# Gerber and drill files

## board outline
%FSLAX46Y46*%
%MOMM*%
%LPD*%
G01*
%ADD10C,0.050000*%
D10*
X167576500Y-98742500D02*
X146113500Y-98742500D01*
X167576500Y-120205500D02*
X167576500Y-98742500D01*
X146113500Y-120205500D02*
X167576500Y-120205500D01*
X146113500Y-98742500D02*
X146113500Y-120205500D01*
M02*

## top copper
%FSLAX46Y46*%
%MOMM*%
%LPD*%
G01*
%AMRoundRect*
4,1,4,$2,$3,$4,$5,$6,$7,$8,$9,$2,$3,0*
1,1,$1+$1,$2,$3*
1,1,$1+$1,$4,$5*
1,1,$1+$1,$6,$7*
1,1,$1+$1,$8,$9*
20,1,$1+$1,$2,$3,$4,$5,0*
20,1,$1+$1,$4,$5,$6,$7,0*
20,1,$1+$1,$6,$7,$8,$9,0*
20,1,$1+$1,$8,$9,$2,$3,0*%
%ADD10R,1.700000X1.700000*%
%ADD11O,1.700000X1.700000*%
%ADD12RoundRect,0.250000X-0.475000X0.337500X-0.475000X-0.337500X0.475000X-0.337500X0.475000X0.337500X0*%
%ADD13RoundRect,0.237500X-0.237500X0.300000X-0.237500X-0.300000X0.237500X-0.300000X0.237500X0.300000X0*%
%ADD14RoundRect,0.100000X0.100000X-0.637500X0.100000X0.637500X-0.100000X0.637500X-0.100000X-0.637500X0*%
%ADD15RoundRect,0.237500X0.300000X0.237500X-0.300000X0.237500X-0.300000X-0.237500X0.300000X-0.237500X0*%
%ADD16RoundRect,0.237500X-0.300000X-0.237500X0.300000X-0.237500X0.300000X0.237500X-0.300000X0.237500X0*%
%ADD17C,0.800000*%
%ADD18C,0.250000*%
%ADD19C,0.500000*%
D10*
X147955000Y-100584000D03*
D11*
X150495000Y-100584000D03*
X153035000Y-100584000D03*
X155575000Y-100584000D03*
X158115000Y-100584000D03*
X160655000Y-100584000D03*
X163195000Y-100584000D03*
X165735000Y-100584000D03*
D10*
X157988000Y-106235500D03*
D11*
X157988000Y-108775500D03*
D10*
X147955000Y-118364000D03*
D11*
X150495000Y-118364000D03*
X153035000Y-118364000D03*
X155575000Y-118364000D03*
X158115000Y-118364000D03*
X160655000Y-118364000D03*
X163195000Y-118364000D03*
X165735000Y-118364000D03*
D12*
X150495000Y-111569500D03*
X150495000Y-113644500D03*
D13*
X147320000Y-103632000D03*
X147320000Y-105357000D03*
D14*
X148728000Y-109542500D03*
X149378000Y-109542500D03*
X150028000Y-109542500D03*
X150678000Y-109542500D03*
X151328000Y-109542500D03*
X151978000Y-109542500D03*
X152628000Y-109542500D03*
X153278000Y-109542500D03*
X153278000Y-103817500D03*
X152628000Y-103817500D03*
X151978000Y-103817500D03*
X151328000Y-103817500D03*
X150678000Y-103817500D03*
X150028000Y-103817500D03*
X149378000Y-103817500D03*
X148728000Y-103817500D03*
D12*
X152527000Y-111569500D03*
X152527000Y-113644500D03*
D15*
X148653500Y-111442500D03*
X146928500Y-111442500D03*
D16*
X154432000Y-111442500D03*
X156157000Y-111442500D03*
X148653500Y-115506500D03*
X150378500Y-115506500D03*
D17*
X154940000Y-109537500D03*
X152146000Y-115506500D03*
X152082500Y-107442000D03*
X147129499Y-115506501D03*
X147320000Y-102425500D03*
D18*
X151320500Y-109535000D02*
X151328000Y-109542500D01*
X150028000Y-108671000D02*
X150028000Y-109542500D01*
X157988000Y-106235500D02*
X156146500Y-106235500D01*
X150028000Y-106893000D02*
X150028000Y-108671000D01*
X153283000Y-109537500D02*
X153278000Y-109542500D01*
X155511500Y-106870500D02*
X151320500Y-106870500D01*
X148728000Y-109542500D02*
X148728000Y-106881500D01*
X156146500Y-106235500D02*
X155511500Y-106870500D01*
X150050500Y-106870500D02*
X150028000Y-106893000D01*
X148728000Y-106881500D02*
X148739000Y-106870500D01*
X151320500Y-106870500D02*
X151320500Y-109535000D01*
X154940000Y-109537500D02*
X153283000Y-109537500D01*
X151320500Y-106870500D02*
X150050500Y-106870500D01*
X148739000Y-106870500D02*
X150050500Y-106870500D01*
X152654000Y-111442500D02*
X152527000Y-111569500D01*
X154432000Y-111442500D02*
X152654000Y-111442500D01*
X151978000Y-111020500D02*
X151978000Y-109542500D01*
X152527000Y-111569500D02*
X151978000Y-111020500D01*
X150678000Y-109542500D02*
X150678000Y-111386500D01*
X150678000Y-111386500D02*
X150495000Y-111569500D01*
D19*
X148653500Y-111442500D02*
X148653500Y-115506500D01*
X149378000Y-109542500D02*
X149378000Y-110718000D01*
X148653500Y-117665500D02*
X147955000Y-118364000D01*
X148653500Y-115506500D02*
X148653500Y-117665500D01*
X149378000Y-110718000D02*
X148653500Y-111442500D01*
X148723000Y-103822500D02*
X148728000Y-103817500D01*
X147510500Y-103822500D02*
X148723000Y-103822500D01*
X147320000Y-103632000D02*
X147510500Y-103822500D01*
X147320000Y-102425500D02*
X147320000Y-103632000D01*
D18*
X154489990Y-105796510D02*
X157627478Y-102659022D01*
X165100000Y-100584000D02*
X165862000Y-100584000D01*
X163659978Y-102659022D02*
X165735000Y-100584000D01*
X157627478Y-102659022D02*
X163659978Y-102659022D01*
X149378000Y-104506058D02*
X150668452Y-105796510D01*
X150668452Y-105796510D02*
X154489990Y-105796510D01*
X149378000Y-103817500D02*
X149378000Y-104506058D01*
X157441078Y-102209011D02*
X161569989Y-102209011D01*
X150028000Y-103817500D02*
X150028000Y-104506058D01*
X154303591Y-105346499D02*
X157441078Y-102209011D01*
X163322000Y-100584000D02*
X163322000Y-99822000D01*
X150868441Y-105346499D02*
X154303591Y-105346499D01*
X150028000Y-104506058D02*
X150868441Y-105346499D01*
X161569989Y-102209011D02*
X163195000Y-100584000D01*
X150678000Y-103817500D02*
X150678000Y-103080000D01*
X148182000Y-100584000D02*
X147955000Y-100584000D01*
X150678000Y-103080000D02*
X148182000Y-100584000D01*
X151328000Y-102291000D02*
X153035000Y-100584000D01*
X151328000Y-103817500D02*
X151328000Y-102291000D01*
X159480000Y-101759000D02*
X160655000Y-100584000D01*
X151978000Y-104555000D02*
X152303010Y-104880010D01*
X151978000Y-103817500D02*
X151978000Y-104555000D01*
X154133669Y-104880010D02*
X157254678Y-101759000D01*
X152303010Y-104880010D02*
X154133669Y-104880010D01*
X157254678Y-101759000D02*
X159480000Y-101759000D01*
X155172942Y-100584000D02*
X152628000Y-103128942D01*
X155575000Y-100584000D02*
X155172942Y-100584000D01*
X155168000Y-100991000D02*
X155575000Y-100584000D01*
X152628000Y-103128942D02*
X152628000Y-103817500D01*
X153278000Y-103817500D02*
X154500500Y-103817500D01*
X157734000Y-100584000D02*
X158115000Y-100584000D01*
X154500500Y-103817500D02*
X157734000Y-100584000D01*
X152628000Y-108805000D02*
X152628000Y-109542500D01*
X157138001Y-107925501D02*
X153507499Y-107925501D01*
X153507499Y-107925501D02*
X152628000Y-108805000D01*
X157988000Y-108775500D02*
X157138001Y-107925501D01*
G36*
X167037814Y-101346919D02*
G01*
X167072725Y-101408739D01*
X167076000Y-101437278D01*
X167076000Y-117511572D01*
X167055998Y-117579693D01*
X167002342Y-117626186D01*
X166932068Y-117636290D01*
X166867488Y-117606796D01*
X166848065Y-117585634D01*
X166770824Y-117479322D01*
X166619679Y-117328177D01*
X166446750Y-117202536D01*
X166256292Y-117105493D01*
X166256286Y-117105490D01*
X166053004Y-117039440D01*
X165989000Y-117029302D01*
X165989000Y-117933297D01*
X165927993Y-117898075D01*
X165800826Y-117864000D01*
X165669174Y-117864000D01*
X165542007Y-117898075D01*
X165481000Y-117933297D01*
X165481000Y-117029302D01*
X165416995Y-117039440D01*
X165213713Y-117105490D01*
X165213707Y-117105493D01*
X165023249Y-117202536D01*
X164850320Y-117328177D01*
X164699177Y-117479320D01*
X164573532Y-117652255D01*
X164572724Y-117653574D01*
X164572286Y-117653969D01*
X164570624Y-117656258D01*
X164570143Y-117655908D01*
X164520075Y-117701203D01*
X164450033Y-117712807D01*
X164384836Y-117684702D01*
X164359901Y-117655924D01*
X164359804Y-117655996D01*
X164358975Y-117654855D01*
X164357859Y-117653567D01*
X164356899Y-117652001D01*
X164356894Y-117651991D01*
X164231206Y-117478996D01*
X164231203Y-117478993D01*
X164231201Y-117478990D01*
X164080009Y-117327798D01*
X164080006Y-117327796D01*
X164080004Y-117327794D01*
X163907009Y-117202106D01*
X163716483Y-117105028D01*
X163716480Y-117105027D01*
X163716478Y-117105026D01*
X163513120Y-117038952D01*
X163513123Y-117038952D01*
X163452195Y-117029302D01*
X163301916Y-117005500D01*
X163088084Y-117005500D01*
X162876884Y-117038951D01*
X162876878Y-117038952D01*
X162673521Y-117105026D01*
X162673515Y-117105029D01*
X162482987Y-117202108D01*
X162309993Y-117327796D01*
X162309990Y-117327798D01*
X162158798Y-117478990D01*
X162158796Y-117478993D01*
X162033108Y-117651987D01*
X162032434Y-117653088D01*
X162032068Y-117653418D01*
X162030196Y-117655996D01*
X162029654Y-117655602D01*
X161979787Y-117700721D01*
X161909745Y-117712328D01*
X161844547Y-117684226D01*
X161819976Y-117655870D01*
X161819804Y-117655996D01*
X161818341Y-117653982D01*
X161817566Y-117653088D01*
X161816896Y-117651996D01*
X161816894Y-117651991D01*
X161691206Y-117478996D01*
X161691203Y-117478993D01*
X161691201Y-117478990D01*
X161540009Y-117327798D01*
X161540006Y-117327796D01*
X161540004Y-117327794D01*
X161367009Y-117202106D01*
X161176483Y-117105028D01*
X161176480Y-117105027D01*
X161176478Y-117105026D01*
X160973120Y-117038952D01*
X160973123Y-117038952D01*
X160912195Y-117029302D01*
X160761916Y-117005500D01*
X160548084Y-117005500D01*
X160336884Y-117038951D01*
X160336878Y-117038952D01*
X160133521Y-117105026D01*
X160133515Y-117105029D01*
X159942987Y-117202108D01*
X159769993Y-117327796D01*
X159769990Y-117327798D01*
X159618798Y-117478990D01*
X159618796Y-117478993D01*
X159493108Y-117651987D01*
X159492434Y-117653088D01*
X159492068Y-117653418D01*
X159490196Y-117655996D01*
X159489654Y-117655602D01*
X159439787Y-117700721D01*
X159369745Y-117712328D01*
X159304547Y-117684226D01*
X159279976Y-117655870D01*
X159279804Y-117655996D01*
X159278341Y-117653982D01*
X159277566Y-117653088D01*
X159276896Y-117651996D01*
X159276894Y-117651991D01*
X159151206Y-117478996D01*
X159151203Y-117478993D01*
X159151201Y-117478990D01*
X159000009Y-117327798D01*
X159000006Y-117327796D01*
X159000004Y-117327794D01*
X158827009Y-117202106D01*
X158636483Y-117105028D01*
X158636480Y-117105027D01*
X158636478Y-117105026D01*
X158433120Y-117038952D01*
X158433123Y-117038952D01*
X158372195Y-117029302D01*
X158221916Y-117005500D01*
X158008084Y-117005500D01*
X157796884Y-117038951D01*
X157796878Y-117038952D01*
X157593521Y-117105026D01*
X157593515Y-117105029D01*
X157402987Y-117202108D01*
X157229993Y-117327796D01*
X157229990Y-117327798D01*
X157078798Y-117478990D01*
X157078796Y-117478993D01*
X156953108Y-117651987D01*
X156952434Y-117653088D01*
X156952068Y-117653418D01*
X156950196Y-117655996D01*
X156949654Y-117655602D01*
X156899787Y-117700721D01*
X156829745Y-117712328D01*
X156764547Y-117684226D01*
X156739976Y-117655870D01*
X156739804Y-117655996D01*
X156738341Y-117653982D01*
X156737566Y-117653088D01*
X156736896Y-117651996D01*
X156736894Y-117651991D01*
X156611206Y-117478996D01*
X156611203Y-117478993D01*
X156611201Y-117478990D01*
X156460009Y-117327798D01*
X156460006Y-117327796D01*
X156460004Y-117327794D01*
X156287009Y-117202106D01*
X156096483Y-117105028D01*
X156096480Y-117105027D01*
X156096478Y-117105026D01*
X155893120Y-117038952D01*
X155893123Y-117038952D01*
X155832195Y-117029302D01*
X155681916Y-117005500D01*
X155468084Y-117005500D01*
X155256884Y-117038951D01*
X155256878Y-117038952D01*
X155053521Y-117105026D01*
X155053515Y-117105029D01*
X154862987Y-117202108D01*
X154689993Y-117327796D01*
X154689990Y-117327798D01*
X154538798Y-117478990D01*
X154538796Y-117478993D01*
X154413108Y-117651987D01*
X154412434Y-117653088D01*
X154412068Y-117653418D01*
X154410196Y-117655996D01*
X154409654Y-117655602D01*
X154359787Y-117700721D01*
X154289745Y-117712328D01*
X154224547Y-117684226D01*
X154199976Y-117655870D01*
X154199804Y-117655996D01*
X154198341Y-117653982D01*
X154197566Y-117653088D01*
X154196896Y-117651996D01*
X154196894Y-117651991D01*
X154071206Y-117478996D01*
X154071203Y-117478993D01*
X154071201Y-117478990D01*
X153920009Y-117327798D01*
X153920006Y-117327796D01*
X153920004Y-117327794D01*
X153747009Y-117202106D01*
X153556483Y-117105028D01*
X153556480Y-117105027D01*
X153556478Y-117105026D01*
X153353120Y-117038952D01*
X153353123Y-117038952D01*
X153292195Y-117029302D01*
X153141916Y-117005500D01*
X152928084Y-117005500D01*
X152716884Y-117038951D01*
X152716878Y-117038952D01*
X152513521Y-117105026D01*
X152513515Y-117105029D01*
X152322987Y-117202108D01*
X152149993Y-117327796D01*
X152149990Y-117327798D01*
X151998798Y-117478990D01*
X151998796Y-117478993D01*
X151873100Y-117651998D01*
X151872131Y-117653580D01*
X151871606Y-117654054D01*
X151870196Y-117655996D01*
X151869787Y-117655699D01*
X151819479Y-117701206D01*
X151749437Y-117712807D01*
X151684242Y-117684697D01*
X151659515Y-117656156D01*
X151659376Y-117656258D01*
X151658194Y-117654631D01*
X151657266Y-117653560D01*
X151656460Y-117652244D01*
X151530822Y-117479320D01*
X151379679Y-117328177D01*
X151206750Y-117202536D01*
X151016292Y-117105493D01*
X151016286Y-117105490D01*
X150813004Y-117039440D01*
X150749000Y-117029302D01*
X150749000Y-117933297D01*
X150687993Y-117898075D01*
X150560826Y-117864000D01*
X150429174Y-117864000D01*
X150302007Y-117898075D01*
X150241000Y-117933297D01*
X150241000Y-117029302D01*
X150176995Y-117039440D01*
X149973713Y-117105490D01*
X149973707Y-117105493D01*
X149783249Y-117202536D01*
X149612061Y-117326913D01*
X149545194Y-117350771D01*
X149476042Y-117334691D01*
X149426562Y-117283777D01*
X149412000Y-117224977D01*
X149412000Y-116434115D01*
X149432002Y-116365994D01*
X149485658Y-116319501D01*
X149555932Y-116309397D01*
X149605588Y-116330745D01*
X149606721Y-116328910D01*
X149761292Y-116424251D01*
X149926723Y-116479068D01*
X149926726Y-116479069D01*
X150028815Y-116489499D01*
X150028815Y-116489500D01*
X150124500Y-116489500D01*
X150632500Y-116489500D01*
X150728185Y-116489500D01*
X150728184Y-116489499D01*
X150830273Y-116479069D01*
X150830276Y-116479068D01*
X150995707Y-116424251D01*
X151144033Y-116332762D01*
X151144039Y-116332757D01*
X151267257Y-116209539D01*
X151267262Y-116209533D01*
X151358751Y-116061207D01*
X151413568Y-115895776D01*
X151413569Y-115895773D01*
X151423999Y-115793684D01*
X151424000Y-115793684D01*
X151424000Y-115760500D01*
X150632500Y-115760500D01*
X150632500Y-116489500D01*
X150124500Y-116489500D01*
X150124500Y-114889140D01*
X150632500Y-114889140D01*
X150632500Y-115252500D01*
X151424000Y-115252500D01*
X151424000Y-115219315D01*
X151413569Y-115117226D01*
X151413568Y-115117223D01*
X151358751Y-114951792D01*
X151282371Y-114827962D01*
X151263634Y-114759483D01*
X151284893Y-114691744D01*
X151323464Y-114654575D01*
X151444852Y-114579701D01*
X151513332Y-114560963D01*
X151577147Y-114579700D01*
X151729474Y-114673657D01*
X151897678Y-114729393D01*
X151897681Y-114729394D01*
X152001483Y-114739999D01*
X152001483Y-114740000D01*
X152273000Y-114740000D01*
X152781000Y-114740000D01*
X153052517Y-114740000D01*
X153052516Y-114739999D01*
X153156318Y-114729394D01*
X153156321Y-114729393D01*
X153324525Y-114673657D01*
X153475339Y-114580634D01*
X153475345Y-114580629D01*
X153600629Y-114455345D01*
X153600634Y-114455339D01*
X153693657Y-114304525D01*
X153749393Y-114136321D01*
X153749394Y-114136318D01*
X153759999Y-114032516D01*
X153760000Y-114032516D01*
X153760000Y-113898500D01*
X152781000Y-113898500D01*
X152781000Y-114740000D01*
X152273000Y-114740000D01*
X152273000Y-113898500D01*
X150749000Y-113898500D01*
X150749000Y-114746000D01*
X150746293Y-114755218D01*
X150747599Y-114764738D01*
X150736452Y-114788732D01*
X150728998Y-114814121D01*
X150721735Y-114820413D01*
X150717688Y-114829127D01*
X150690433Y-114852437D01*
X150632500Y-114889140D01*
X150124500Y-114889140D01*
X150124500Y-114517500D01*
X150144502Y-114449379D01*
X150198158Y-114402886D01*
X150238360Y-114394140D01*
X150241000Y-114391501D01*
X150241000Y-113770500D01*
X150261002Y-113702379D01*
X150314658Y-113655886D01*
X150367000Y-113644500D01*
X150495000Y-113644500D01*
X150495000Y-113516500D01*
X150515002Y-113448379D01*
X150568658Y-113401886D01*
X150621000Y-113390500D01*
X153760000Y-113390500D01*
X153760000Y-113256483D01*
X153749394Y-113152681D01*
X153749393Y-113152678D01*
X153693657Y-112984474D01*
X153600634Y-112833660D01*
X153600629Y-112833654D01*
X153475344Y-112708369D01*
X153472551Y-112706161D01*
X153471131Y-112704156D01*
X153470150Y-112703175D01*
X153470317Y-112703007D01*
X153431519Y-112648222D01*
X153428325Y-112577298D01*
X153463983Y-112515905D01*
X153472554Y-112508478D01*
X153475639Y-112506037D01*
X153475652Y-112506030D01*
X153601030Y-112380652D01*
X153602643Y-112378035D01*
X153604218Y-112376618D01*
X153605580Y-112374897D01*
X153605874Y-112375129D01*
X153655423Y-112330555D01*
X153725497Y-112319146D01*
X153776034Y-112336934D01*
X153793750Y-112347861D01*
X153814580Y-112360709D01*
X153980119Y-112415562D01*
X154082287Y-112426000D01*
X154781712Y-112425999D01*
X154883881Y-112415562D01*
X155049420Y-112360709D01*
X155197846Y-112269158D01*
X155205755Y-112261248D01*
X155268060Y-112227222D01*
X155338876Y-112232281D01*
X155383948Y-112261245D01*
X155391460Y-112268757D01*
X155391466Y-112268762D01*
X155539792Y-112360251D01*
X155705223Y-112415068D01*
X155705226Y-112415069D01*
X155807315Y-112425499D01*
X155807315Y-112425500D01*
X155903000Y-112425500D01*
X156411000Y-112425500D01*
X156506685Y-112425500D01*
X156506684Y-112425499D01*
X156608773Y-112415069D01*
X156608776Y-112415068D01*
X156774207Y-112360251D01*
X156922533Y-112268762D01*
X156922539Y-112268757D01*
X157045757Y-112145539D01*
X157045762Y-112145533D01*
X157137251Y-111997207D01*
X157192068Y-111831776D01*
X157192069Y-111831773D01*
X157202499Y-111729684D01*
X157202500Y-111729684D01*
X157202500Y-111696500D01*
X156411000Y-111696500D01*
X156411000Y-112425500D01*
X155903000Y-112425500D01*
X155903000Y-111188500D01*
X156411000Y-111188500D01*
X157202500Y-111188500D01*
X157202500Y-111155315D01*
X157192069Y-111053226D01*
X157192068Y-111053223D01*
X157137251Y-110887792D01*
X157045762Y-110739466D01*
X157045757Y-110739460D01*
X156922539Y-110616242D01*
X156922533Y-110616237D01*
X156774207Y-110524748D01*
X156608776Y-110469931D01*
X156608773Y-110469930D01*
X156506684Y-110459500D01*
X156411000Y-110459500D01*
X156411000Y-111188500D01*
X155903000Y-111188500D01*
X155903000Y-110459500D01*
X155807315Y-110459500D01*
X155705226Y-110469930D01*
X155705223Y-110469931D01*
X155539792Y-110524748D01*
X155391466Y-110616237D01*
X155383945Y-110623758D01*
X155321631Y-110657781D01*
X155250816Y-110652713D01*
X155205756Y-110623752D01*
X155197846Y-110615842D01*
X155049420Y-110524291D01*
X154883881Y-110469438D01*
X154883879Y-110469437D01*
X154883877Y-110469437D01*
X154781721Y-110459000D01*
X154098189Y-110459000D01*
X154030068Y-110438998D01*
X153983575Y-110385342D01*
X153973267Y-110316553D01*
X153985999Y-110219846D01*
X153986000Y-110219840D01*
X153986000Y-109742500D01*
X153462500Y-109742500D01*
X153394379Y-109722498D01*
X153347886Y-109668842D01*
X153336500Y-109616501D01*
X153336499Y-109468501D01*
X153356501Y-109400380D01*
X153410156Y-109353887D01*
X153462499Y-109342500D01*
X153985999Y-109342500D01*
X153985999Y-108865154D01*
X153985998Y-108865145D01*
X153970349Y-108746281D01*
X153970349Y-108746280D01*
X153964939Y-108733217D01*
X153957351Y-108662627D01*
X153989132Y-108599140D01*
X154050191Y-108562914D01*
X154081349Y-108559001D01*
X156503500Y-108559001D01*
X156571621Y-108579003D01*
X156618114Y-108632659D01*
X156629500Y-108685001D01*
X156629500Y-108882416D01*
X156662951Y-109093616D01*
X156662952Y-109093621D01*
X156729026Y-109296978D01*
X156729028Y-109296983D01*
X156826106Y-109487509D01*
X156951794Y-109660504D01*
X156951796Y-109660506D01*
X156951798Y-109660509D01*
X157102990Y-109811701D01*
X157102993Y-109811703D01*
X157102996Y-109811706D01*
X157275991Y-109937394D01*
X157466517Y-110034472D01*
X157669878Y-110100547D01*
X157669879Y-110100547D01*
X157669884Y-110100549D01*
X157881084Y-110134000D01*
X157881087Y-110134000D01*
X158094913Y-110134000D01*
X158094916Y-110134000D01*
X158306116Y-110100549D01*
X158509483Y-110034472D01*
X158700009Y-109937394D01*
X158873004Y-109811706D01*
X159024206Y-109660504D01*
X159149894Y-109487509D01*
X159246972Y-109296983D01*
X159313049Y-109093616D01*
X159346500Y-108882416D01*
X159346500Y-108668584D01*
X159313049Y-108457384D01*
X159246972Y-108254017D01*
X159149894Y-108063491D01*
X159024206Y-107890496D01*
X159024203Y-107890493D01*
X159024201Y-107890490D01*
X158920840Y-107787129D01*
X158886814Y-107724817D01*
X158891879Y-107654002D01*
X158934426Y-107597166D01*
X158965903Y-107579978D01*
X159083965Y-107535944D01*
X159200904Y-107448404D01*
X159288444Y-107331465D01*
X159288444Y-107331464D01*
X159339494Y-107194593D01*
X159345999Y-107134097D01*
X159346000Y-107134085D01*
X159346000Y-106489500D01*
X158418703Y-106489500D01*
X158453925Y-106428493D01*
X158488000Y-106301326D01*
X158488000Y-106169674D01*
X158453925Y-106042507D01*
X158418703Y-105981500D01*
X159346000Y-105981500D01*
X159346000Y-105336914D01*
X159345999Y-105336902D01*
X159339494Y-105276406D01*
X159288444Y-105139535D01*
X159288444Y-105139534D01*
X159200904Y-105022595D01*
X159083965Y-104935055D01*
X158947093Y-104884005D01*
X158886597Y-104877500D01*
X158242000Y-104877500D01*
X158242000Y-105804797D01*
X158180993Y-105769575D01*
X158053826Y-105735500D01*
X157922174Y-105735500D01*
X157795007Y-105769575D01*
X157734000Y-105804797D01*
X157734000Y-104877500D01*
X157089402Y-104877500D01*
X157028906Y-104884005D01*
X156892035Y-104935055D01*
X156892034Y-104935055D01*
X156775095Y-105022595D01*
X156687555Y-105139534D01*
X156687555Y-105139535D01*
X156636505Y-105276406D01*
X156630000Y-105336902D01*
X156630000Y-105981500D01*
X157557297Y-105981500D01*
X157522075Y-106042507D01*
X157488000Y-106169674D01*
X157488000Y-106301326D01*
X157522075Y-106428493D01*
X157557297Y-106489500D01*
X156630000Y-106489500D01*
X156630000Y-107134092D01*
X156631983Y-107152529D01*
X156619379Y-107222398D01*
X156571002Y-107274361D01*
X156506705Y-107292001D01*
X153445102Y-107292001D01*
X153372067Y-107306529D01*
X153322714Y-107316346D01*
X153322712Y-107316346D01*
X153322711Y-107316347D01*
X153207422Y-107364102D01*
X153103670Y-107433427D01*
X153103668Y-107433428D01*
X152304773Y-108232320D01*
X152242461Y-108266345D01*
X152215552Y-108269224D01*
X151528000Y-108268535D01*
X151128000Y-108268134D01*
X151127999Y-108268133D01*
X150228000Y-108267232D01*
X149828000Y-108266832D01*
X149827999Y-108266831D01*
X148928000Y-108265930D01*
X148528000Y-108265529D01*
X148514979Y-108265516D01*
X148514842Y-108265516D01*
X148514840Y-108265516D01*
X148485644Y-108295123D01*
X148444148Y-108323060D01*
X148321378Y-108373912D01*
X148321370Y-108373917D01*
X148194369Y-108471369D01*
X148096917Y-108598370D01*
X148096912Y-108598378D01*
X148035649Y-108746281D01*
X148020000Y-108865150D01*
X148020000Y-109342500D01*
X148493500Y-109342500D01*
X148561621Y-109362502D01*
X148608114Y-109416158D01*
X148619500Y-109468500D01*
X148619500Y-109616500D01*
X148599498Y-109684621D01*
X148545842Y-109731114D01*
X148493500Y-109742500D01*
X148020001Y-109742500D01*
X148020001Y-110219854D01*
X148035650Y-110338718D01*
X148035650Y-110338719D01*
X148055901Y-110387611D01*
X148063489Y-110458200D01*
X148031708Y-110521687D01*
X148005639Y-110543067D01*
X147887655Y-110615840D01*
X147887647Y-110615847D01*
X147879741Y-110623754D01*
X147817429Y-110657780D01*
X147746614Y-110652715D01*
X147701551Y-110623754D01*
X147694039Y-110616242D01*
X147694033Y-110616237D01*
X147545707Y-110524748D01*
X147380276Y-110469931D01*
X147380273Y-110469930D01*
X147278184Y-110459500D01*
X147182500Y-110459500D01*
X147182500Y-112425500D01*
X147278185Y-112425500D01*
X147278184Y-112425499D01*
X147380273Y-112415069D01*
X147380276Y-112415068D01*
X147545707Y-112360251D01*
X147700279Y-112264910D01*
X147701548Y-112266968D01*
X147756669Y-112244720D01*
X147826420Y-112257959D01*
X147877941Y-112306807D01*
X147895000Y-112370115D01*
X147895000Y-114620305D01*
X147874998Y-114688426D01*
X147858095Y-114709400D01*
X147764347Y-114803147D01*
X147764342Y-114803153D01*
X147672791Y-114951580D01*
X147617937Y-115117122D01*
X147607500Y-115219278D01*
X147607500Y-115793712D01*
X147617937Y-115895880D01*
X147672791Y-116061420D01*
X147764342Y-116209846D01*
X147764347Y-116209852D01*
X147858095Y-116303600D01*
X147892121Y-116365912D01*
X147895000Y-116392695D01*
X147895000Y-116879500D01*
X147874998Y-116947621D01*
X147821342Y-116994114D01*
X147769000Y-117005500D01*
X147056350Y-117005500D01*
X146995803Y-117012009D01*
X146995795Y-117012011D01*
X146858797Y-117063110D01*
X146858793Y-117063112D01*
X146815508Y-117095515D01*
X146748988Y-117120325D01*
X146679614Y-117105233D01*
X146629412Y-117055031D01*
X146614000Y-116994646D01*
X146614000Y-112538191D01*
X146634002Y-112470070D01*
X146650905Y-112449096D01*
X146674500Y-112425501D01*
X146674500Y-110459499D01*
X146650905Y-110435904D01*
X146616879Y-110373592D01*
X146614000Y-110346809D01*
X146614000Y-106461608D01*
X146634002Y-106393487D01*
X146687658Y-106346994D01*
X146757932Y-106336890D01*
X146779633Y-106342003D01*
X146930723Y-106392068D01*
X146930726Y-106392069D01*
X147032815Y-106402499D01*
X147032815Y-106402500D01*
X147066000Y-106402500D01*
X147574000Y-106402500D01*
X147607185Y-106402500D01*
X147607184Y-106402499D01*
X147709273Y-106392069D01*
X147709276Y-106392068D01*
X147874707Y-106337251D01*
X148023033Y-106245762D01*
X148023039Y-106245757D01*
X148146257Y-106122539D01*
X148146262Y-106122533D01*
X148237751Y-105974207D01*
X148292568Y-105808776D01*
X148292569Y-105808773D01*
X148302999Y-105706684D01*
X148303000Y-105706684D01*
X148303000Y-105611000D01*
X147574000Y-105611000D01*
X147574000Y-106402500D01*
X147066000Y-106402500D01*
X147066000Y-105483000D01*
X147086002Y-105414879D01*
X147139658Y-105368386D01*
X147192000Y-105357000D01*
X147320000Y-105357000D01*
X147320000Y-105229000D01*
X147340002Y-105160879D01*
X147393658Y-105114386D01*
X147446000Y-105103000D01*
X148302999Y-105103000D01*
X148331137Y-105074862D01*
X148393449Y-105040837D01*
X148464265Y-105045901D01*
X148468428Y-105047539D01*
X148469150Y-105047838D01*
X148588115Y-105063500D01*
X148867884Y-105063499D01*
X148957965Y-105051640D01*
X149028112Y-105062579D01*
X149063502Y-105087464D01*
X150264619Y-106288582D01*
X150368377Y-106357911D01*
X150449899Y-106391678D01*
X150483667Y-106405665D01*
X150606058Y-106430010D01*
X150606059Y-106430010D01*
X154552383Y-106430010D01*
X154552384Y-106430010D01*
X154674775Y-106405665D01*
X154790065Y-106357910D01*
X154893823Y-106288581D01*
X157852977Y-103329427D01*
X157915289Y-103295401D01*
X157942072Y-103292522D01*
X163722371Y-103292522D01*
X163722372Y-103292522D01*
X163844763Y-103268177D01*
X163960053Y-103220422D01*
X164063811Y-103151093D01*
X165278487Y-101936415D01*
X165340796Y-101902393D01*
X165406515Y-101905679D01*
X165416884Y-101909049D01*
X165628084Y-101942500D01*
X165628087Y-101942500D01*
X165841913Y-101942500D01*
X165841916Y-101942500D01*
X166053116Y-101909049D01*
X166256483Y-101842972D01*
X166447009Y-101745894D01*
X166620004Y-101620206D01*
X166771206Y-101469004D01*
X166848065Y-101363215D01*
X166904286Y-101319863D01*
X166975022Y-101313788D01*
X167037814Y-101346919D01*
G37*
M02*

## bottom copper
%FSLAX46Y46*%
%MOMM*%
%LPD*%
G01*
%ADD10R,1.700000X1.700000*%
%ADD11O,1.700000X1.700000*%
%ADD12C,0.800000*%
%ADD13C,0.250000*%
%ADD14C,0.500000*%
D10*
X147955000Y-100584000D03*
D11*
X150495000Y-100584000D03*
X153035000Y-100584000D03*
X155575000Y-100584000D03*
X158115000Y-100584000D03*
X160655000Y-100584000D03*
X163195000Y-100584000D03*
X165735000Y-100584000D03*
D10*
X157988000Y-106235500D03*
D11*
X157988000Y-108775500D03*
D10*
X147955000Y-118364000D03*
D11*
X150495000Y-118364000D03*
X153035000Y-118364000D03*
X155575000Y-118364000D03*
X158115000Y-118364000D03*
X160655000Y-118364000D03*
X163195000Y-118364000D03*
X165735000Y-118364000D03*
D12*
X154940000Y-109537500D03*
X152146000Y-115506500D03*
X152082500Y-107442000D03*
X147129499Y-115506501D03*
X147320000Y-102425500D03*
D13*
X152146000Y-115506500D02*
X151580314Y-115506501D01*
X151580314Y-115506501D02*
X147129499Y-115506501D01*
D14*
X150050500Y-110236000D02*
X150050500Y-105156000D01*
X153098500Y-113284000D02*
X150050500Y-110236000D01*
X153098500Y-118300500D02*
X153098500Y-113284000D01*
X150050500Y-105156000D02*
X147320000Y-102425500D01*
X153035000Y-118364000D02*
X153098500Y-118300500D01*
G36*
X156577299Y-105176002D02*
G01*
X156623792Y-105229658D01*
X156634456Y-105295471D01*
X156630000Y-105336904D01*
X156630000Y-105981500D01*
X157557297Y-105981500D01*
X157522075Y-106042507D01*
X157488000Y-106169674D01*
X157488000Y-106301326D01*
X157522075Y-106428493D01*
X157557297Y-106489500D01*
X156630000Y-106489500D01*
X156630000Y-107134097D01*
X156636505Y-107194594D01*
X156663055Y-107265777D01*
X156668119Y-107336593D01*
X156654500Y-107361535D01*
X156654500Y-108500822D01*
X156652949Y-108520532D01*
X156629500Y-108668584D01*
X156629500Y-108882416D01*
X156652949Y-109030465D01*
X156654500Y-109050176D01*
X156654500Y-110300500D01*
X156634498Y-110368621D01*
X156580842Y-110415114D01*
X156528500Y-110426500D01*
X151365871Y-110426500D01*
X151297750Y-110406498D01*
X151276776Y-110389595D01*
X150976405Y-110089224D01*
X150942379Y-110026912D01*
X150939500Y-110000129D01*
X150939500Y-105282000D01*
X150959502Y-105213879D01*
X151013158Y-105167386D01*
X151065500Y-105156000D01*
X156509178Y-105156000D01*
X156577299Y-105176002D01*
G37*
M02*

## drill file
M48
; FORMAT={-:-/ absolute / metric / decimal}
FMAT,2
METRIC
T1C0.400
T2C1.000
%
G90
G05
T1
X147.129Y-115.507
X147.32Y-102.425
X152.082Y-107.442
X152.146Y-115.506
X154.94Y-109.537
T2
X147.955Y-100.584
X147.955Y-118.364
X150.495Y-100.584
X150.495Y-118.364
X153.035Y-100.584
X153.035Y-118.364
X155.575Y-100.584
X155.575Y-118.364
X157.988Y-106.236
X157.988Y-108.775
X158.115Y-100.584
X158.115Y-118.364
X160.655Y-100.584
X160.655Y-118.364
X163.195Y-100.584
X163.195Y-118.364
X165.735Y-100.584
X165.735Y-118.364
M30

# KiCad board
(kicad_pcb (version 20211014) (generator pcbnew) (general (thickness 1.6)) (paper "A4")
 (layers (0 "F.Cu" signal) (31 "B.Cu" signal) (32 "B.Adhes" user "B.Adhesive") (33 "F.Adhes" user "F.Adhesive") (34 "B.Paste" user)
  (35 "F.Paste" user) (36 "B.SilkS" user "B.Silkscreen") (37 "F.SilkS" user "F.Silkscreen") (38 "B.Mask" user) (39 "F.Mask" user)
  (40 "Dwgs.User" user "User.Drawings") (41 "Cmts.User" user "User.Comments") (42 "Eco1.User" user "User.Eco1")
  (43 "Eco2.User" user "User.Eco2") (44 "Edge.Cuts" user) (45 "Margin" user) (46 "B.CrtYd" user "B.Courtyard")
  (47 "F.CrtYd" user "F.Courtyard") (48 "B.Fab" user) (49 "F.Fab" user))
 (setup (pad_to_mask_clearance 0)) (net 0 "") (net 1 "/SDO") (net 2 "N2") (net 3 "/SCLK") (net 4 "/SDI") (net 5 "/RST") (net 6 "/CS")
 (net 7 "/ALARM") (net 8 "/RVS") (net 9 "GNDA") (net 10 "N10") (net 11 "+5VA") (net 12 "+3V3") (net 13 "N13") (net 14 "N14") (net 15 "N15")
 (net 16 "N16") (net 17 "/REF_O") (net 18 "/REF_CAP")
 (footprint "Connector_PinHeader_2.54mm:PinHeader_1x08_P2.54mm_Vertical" (layer "F.Cu") (at 147.955 100.584 90)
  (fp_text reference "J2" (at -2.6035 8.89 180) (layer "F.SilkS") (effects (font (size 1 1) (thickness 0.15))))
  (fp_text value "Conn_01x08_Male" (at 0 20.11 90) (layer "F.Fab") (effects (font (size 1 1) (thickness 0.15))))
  (pad "1" thru_hole rect locked (at 0 0 90) (size 1.7 1.7) (drill 1) (layers *.Cu *.Mask) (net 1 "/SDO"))
  (pad "2" thru_hole oval locked (at 0 2.54 90) (size 1.7 1.7) (drill 1) (layers *.Cu *.Mask) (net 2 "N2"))
  (pad "3" thru_hole oval locked (at 0 5.08 90) (size 1.7 1.7) (drill 1) (layers *.Cu *.Mask) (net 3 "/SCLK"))
  (pad "4" thru_hole oval locked (at 0 7.62 90) (size 1.7 1.7) (drill 1) (layers *.Cu *.Mask) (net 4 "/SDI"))
  (pad "5" thru_hole oval locked (at 0 10.16 90) (size 1.7 1.7) (drill 1) (layers *.Cu *.Mask) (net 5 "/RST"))
  (pad "6" thru_hole oval locked (at 0 12.7 90) (size 1.7 1.7) (drill 1) (layers *.Cu *.Mask) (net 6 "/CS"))
  (pad "7" thru_hole oval locked (at 0 15.24 90) (size 1.7 1.7) (drill 1) (layers *.Cu *.Mask) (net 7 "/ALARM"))
  (pad "8" thru_hole oval locked (at 0 17.78 90) (size 1.7 1.7) (drill 1) (layers *.Cu *.Mask) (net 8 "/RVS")))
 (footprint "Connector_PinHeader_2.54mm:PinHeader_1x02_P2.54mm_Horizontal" (layer "F.Cu") (at 157.988 106.2355)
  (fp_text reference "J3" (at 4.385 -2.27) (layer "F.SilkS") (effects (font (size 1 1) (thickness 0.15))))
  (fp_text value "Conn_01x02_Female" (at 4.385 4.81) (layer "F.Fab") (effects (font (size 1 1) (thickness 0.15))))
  (pad "1" thru_hole rect locked (at 0 0) (size 1.7 1.7) (drill 1) (layers *.Cu *.Mask) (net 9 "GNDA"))
  (pad "2" thru_hole oval locked (at 0 2.54) (size 1.7 1.7) (drill 1) (layers *.Cu *.Mask) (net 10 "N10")))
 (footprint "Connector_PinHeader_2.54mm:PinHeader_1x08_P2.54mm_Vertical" (layer "F.Cu") (at 147.955 118.364 90)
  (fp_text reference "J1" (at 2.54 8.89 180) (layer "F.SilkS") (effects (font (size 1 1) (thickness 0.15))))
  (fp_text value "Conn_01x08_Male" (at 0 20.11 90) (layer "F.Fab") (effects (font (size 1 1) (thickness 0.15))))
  (pad "1" thru_hole rect locked (at 0 0 90) (size 1.7 1.7) (drill 1) (layers *.Cu *.Mask) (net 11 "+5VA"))
  (pad "2" thru_hole oval locked (at 0 2.54 90) (size 1.7 1.7) (drill 1) (layers *.Cu *.Mask) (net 9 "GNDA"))
  (pad "3" thru_hole oval locked (at 0 5.08 90) (size 1.7 1.7) (drill 1) (layers *.Cu *.Mask) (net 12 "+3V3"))
  (pad "4" thru_hole oval locked (at 0 7.62 90) (size 1.7 1.7) (drill 1) (layers *.Cu *.Mask) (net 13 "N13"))
  (pad "5" thru_hole oval locked (at 0 10.16 90) (size 1.7 1.7) (drill 1) (layers *.Cu *.Mask) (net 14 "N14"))
  (pad "6" thru_hole oval locked (at 0 12.7 90) (size 1.7 1.7) (drill 1) (layers *.Cu *.Mask) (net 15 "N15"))
  (pad "7" thru_hole oval locked (at 0 15.24 90) (size 1.7 1.7) (drill 1) (layers *.Cu *.Mask) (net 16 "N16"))
  (pad "8" thru_hole oval locked (at 0 17.78 90) (size 1.7 1.7) (drill 1) (layers *.Cu *.Mask) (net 9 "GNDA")))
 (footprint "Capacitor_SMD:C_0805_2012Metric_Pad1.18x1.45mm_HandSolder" (layer "F.Cu") (at 150.495 112.607 -90)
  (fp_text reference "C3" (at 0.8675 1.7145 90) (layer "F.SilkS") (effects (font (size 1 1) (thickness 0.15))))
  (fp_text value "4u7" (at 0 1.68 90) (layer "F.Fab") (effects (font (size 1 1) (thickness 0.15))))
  (pad "1" smd roundrect locked (at -1.0375 0 270) (size 1.175 1.45) (layers "F.Cu" "F.Paste" "F.Mask") (roundrect_rratio 0.2127659574)
   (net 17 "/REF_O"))
  (pad "2" smd roundrect locked (at 1.0375 0 270) (size 1.175 1.45) (layers "F.Cu" "F.Paste" "F.Mask") (roundrect_rratio 0.2127659574)
   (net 9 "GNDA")))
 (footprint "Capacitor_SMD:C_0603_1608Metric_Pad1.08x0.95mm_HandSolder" (layer "F.Cu") (at 147.32 104.4945 -90)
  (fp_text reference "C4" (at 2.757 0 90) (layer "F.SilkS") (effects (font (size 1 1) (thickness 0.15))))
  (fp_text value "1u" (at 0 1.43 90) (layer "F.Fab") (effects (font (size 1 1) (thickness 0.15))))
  (pad "1" smd roundrect locked (at -0.8625 0 270) (size 1.075 0.95) (layers "F.Cu" "F.Paste" "F.Mask") (roundrect_rratio 0.25)
   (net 12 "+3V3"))
  (pad "2" smd roundrect locked (at 0.8625 0 270) (size 1.075 0.95) (layers "F.Cu" "F.Paste" "F.Mask") (roundrect_rratio 0.25)
   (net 9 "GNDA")))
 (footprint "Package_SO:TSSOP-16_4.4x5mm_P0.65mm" (layer "F.Cu") (at 151.003 106.68 90)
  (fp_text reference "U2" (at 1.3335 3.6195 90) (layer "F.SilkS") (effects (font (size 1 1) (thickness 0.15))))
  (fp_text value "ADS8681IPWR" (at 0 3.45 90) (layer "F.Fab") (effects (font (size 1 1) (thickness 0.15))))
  (pad "1" smd roundrect locked (at -2.8625 -2.275 90) (size 1.475 0.4) (layers "F.Cu" "F.Paste" "F.Mask") (roundrect_rratio 0.25)
   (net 9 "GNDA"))
  (pad "2" smd roundrect locked (at -2.8625 -1.625 90) (size 1.475 0.4) (layers "F.Cu" "F.Paste" "F.Mask") (roundrect_rratio 0.25)
   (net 11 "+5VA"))
  (pad "3" smd roundrect locked (at -2.8625 -0.975 90) (size 1.475 0.4) (layers "F.Cu" "F.Paste" "F.Mask") (roundrect_rratio 0.25)
   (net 9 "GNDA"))
  (pad "4" smd roundrect locked (at -2.8625 -0.325 90) (size 1.475 0.4) (layers "F.Cu" "F.Paste" "F.Mask") (roundrect_rratio 0.25)
   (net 17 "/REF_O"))
  (pad "5" smd roundrect locked (at -2.8625 0.325 90) (size 1.475 0.4) (layers "F.Cu" "F.Paste" "F.Mask") (roundrect_rratio 0.25)
   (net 9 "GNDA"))
  (pad "6" smd roundrect locked (at -2.8625 0.975 90) (size 1.475 0.4) (layers "F.Cu" "F.Paste" "F.Mask") (roundrect_rratio 0.25)
   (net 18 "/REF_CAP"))
  (pad "7" smd roundrect locked (at -2.8625 1.625 90) (size 1.475 0.4) (layers "F.Cu" "F.Paste" "F.Mask") (roundrect_rratio 0.25)
   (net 10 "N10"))
  (pad "8" smd roundrect locked (at -2.8625 2.275 90) (size 1.475 0.4) (layers "F.Cu" "F.Paste" "F.Mask") (roundrect_rratio 0.25)
   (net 9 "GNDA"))
  (pad "9" smd roundrect locked (at 2.8625 2.275 90) (size 1.475 0.4) (layers "F.Cu" "F.Paste" "F.Mask") (roundrect_rratio 0.25)
   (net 5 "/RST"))
  (pad "10" smd roundrect locked (at 2.8625 1.625 90) (size 1.475 0.4) (layers "F.Cu" "F.Paste" "F.Mask") (roundrect_rratio 0.25)
   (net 4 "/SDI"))
  (pad "11" smd roundrect locked (at 2.8625 0.975 90) (size 1.475 0.4) (layers "F.Cu" "F.Paste" "F.Mask") (roundrect_rratio 0.25)
   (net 6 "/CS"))
  (pad "12" smd roundrect locked (at 2.8625 0.325 90) (size 1.475 0.4) (layers "F.Cu" "F.Paste" "F.Mask") (roundrect_rratio 0.25)
   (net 3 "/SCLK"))
  (pad "13" smd roundrect locked (at 2.8625 -0.325 90) (size 1.475 0.4) (layers "F.Cu" "F.Paste" "F.Mask") (roundrect_rratio 0.25)
   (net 1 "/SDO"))
  (pad "14" smd roundrect locked (at 2.8625 -0.975 90) (size 1.475 0.4) (layers "F.Cu" "F.Paste" "F.Mask") (roundrect_rratio 0.25)
   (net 7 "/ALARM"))
  (pad "15" smd roundrect locked (at 2.8625 -1.625 90) (size 1.475 0.4) (layers "F.Cu" "F.Paste" "F.Mask") (roundrect_rratio 0.25)
   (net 8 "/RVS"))
  (pad "16" smd roundrect locked (at 2.8625 -2.275 90) (size 1.475 0.4) (layers "F.Cu" "F.Paste" "F.Mask") (roundrect_rratio 0.25)
   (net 12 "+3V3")))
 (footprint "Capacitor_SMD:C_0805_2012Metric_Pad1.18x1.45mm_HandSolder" (layer "F.Cu") (at 152.527 112.607 -90)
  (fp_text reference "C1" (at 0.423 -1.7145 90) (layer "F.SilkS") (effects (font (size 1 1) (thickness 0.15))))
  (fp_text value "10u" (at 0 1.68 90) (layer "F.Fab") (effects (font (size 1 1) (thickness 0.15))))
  (pad "1" smd roundrect locked (at -1.0375 0 270) (size 1.175 1.45) (layers "F.Cu" "F.Paste" "F.Mask") (roundrect_rratio 0.2127659574)
   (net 18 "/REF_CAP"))
  (pad "2" smd roundrect locked (at 1.0375 0 270) (size 1.175 1.45) (layers "F.Cu" "F.Paste" "F.Mask") (roundrect_rratio 0.2127659574)
   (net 9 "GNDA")))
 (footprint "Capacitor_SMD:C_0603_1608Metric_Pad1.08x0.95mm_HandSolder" (layer "F.Cu") (at 147.791 111.4425 180)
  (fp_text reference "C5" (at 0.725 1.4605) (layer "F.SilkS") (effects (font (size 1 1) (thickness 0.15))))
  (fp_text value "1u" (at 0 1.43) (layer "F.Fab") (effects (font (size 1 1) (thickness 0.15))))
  (pad "1" smd roundrect locked (at -0.8625 0 180) (size 1.075 0.95) (layers "F.Cu" "F.Paste" "F.Mask") (roundrect_rratio 0.25)
   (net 11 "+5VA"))
  (pad "2" smd roundrect locked (at 0.8625 0 180) (size 1.075 0.95) (layers "F.Cu" "F.Paste" "F.Mask") (roundrect_rratio 0.25)
   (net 9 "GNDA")))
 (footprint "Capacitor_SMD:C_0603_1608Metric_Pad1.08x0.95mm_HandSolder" (layer "F.Cu") (at 155.2945 111.4425)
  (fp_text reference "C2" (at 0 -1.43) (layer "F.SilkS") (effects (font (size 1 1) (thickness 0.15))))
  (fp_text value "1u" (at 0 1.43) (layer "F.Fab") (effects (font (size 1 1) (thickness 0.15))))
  (pad "1" smd roundrect locked (at -0.8625 0) (size 1.075 0.95) (layers "F.Cu" "F.Paste" "F.Mask") (roundrect_rratio 0.25)
   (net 18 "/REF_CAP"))
  (pad "2" smd roundrect locked (at 0.8625 0) (size 1.075 0.95) (layers "F.Cu" "F.Paste" "F.Mask") (roundrect_rratio 0.25) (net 9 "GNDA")))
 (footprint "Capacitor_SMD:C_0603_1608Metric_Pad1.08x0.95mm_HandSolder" (layer "F.Cu") (at 149.516 115.5065)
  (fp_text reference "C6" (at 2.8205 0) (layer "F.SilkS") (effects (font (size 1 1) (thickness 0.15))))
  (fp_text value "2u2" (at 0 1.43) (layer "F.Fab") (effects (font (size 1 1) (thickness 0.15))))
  (pad "1" smd roundrect locked (at -0.8625 0) (size 1.075 0.95) (layers "F.Cu" "F.Paste" "F.Mask") (roundrect_rratio 0.25) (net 11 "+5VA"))
  (pad "2" smd roundrect locked (at 0.8625 0) (size 1.075 0.95) (layers "F.Cu" "F.Paste" "F.Mask") (roundrect_rratio 0.25) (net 9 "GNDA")))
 (gr_line (start 167.5765 98.7425) (end 146.1135 98.7425) (layer "Edge.Cuts") (width 0.05))
 (gr_line (start 167.5765 120.2055) (end 167.5765 98.7425) (layer "Edge.Cuts") (width 0.05))
 (gr_line (start 146.1135 120.2055) (end 167.5765 120.2055) (layer "Edge.Cuts") (width 0.05))
 (gr_line (start 146.1135 98.7425) (end 146.1135 120.2055) (layer "Edge.Cuts") (width 0.05))
 (segment (start 151.3205 109.535) (end 151.328 109.5425) (width 0.25) (layer "F.Cu") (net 9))
 (segment (start 150.028 108.671) (end 150.028 109.5425) (width 0.25) (layer "F.Cu") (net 9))
 (segment (start 157.988 106.2355) (end 156.1465 106.2355) (width 0.25) (layer "F.Cu") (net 9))
 (segment (start 150.028 106.893) (end 150.028 108.671) (width 0.25) (layer "F.Cu") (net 9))
 (segment (start 153.283 109.5375) (end 153.278 109.5425) (width 0.25) (layer "F.Cu") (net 9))
 (segment (start 155.5115 106.8705) (end 151.3205 106.8705) (width 0.25) (layer "F.Cu") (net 9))
 (segment (start 148.728 109.5425) (end 148.728 106.8815) (width 0.25) (layer "F.Cu") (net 9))
 (segment (start 156.1465 106.2355) (end 155.5115 106.8705) (width 0.25) (layer "F.Cu") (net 9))
 (segment (start 150.0505 106.8705) (end 150.028 106.893) (width 0.25) (layer "F.Cu") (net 9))
 (segment (start 148.728 106.8815) (end 148.739 106.8705) (width 0.25) (layer "F.Cu") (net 9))
 (segment (start 151.3205 106.8705) (end 151.3205 109.535) (width 0.25) (layer "F.Cu") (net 9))
 (segment (start 154.94 109.5375) (end 153.283 109.5375) (width 0.25) (layer "F.Cu") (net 9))
 (segment (start 151.3205 106.8705) (end 150.0505 106.8705) (width 0.25) (layer "F.Cu") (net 9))
 (segment (start 148.739 106.8705) (end 150.0505 106.8705) (width 0.25) (layer "F.Cu") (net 9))
 (via (at 154.94 109.5375) (size 0.8) (drill 0.4) (layers "F.Cu" "B.Cu") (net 9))
 (via (at 152.146 115.5065) (size 0.8) (drill 0.4) (layers "F.Cu" "B.Cu") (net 9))
 (via (at 152.0825 107.442) (size 0.8) (drill 0.4) (layers "F.Cu" "B.Cu") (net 9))
 (via (at 147.129499 115.506501) (size 0.8) (drill 0.4) (layers "F.Cu" "B.Cu") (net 9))
 (segment (start 152.146 115.5065) (end 151.580314 115.506501) (width 0.25) (layer "B.Cu") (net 9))
 (segment (start 151.580314 115.506501) (end 147.129499 115.506501) (width 0.25) (layer "B.Cu") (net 9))
 (segment (start 152.654 111.4425) (end 152.527 111.5695) (width 0.25) (layer "F.Cu") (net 18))
 (segment (start 154.432 111.4425) (end 152.654 111.4425) (width 0.25) (layer "F.Cu") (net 18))
 (segment (start 151.978 111.0205) (end 151.978 109.5425) (width 0.25) (layer "F.Cu") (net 18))
 (segment (start 152.527 111.5695) (end 151.978 111.0205) (width 0.25) (layer "F.Cu") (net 18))
 (segment (start 150.678 109.5425) (end 150.678 111.3865) (width 0.25) (layer "F.Cu") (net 17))
 (segment (start 150.678 111.3865) (end 150.495 111.5695) (width 0.25) (layer "F.Cu") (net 17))
 (segment (start 148.6535 111.4425) (end 148.6535 115.5065) (width 0.5) (layer "F.Cu") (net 11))
 (segment (start 149.378 109.5425) (end 149.378 110.718) (width 0.5) (layer "F.Cu") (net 11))
 (segment (start 148.6535 117.6655) (end 147.955 118.364) (width 0.5) (layer "F.Cu") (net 11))
 (segment (start 148.6535 115.5065) (end 148.6535 117.6655) (width 0.5) (layer "F.Cu") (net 11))
 (segment (start 149.378 110.718) (end 148.6535 111.4425) (width 0.5) (layer "F.Cu") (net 11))
 (segment (start 148.723 103.8225) (end 148.728 103.8175) (width 0.5) (layer "F.Cu") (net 12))
 (segment (start 147.5105 103.8225) (end 148.723 103.8225) (width 0.5) (layer "F.Cu") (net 12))
 (segment (start 147.32 103.632) (end 147.5105 103.8225) (width 0.5) (layer "F.Cu") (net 12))
 (segment (start 147.32 102.4255) (end 147.32 103.632) (width 0.5) (layer "F.Cu") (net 12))
 (via (at 147.32 102.4255) (size 0.8) (drill 0.4) (layers "F.Cu" "B.Cu") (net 12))
 (segment (start 150.0505 110.236) (end 150.0505 105.156) (width 0.5) (layer "B.Cu") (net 12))
 (segment (start 153.0985 113.284) (end 150.0505 110.236) (width 0.5) (layer "B.Cu") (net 12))
 (segment (start 153.0985 118.3005) (end 153.0985 113.284) (width 0.5) (layer "B.Cu") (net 12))
 (segment (start 150.0505 105.156) (end 147.32 102.4255) (width 0.5) (layer "B.Cu") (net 12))
 (segment (start 153.035 118.364) (end 153.0985 118.3005) (width 0.5) (layer "B.Cu") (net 12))
 (segment (start 154.48999 105.79651) (end 157.627478 102.659022) (width 0.25) (layer "F.Cu") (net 8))
 (segment (start 165.1 100.584) (end 165.862 100.584) (width 0.25) (layer "F.Cu") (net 8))
 (segment (start 163.659978 102.659022) (end 165.735 100.584) (width 0.25) (layer "F.Cu") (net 8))
 (segment (start 157.627478 102.659022) (end 163.659978 102.659022) (width 0.25) (layer "F.Cu") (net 8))
 (segment (start 149.378 104.506058) (end 150.668452 105.79651) (width 0.25) (layer "F.Cu") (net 8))
 (segment (start 150.668452 105.79651) (end 154.48999 105.79651) (width 0.25) (layer "F.Cu") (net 8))
 (segment (start 149.378 103.8175) (end 149.378 104.506058) (width 0.25) (layer "F.Cu") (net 8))
 (segment (start 157.441078 102.209011) (end 161.569989 102.209011) (width 0.25) (layer "F.Cu") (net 7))
 (segment (start 150.028 103.8175) (end 150.028 104.506058) (width 0.25) (layer "F.Cu") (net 7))
 (segment (start 154.303591 105.346499) (end 157.441078 102.209011) (width 0.25) (layer "F.Cu") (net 7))
 (segment (start 163.322 100.584) (end 163.322 99.822) (width 0.25) (layer "F.Cu") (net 7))
 (segment (start 150.868441 105.346499) (end 154.303591 105.346499) (width 0.25) (layer "F.Cu") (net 7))
 (segment (start 150.028 104.506058) (end 150.868441 105.346499) (width 0.25) (layer "F.Cu") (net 7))
 (segment (start 161.569989 102.209011) (end 163.195 100.584) (width 0.25) (layer "F.Cu") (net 7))
 (segment (start 150.678 103.8175) (end 150.678 103.08) (width 0.25) (layer "F.Cu") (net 1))
 (segment (start 148.182 100.584) (end 147.955 100.584) (width 0.25) (layer "F.Cu") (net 1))
 (segment (start 150.678 103.08) (end 148.182 100.584) (width 0.25) (layer "F.Cu") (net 1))
 (segment (start 151.328 102.291) (end 153.035 100.584) (width 0.25) (layer "F.Cu") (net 3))
 (segment (start 151.328 103.8175) (end 151.328 102.291) (width 0.25) (layer "F.Cu") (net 3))
 (segment (start 159.48 101.759) (end 160.655 100.584) (width 0.25) (layer "F.Cu") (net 6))
 (segment (start 151.978 104.555) (end 152.30301 104.88001) (width 0.25) (layer "F.Cu") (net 6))
 (segment (start 151.978 103.8175) (end 151.978 104.555) (width 0.25) (layer "F.Cu") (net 6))
 (segment (start 154.133669 104.88001) (end 157.254678 101.759) (width 0.25) (layer "F.Cu") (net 6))
 (segment (start 152.30301 104.88001) (end 154.133669 104.88001) (width 0.25) (layer "F.Cu") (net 6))
 (segment (start 157.254678 101.759) (end 159.48 101.759) (width 0.25) (layer "F.Cu") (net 6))
 (segment (start 155.172942 100.584) (end 152.628 103.128942) (width 0.25) (layer "F.Cu") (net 4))
 (segment (start 155.575 100.584) (end 155.172942 100.584) (width 0.25) (layer "F.Cu") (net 4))
 (segment (start 155.168 100.991) (end 155.575 100.584) (width 0.25) (layer "F.Cu") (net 4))
 (segment (start 152.628 103.128942) (end 152.628 103.8175) (width 0.25) (layer "F.Cu") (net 4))
 (segment (start 153.278 103.8175) (end 154.5005 103.8175) (width 0.25) (layer "F.Cu") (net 5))
 (segment (start 157.734 100.584) (end 158.115 100.584) (width 0.25) (layer "F.Cu") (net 5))
 (segment (start 154.5005 103.8175) (end 157.734 100.584) (width 0.25) (layer "F.Cu") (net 5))
 (segment (start 152.628 108.805) (end 152.628 109.5425) (width 0.25) (layer "F.Cu") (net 10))
 (segment (start 157.138001 107.925501) (end 153.507499 107.925501) (width 0.25) (layer "F.Cu") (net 10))
 (segment (start 153.507499 107.925501) (end 152.628 108.805) (width 0.25) (layer "F.Cu") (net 10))
 (segment (start 157.988 108.7755) (end 157.138001 107.925501) (width 0.25) (layer "F.Cu") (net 10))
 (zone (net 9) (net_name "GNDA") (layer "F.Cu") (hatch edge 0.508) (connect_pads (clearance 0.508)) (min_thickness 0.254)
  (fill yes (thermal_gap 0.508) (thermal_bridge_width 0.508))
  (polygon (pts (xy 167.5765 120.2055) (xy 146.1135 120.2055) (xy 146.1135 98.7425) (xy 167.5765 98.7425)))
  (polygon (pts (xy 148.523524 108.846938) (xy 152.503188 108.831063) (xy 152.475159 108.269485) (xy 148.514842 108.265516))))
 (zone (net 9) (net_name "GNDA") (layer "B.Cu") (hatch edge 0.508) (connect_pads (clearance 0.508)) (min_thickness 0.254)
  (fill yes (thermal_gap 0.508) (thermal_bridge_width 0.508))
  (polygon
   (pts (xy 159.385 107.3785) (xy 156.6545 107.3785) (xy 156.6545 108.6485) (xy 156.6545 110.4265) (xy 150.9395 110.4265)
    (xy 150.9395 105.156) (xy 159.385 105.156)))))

